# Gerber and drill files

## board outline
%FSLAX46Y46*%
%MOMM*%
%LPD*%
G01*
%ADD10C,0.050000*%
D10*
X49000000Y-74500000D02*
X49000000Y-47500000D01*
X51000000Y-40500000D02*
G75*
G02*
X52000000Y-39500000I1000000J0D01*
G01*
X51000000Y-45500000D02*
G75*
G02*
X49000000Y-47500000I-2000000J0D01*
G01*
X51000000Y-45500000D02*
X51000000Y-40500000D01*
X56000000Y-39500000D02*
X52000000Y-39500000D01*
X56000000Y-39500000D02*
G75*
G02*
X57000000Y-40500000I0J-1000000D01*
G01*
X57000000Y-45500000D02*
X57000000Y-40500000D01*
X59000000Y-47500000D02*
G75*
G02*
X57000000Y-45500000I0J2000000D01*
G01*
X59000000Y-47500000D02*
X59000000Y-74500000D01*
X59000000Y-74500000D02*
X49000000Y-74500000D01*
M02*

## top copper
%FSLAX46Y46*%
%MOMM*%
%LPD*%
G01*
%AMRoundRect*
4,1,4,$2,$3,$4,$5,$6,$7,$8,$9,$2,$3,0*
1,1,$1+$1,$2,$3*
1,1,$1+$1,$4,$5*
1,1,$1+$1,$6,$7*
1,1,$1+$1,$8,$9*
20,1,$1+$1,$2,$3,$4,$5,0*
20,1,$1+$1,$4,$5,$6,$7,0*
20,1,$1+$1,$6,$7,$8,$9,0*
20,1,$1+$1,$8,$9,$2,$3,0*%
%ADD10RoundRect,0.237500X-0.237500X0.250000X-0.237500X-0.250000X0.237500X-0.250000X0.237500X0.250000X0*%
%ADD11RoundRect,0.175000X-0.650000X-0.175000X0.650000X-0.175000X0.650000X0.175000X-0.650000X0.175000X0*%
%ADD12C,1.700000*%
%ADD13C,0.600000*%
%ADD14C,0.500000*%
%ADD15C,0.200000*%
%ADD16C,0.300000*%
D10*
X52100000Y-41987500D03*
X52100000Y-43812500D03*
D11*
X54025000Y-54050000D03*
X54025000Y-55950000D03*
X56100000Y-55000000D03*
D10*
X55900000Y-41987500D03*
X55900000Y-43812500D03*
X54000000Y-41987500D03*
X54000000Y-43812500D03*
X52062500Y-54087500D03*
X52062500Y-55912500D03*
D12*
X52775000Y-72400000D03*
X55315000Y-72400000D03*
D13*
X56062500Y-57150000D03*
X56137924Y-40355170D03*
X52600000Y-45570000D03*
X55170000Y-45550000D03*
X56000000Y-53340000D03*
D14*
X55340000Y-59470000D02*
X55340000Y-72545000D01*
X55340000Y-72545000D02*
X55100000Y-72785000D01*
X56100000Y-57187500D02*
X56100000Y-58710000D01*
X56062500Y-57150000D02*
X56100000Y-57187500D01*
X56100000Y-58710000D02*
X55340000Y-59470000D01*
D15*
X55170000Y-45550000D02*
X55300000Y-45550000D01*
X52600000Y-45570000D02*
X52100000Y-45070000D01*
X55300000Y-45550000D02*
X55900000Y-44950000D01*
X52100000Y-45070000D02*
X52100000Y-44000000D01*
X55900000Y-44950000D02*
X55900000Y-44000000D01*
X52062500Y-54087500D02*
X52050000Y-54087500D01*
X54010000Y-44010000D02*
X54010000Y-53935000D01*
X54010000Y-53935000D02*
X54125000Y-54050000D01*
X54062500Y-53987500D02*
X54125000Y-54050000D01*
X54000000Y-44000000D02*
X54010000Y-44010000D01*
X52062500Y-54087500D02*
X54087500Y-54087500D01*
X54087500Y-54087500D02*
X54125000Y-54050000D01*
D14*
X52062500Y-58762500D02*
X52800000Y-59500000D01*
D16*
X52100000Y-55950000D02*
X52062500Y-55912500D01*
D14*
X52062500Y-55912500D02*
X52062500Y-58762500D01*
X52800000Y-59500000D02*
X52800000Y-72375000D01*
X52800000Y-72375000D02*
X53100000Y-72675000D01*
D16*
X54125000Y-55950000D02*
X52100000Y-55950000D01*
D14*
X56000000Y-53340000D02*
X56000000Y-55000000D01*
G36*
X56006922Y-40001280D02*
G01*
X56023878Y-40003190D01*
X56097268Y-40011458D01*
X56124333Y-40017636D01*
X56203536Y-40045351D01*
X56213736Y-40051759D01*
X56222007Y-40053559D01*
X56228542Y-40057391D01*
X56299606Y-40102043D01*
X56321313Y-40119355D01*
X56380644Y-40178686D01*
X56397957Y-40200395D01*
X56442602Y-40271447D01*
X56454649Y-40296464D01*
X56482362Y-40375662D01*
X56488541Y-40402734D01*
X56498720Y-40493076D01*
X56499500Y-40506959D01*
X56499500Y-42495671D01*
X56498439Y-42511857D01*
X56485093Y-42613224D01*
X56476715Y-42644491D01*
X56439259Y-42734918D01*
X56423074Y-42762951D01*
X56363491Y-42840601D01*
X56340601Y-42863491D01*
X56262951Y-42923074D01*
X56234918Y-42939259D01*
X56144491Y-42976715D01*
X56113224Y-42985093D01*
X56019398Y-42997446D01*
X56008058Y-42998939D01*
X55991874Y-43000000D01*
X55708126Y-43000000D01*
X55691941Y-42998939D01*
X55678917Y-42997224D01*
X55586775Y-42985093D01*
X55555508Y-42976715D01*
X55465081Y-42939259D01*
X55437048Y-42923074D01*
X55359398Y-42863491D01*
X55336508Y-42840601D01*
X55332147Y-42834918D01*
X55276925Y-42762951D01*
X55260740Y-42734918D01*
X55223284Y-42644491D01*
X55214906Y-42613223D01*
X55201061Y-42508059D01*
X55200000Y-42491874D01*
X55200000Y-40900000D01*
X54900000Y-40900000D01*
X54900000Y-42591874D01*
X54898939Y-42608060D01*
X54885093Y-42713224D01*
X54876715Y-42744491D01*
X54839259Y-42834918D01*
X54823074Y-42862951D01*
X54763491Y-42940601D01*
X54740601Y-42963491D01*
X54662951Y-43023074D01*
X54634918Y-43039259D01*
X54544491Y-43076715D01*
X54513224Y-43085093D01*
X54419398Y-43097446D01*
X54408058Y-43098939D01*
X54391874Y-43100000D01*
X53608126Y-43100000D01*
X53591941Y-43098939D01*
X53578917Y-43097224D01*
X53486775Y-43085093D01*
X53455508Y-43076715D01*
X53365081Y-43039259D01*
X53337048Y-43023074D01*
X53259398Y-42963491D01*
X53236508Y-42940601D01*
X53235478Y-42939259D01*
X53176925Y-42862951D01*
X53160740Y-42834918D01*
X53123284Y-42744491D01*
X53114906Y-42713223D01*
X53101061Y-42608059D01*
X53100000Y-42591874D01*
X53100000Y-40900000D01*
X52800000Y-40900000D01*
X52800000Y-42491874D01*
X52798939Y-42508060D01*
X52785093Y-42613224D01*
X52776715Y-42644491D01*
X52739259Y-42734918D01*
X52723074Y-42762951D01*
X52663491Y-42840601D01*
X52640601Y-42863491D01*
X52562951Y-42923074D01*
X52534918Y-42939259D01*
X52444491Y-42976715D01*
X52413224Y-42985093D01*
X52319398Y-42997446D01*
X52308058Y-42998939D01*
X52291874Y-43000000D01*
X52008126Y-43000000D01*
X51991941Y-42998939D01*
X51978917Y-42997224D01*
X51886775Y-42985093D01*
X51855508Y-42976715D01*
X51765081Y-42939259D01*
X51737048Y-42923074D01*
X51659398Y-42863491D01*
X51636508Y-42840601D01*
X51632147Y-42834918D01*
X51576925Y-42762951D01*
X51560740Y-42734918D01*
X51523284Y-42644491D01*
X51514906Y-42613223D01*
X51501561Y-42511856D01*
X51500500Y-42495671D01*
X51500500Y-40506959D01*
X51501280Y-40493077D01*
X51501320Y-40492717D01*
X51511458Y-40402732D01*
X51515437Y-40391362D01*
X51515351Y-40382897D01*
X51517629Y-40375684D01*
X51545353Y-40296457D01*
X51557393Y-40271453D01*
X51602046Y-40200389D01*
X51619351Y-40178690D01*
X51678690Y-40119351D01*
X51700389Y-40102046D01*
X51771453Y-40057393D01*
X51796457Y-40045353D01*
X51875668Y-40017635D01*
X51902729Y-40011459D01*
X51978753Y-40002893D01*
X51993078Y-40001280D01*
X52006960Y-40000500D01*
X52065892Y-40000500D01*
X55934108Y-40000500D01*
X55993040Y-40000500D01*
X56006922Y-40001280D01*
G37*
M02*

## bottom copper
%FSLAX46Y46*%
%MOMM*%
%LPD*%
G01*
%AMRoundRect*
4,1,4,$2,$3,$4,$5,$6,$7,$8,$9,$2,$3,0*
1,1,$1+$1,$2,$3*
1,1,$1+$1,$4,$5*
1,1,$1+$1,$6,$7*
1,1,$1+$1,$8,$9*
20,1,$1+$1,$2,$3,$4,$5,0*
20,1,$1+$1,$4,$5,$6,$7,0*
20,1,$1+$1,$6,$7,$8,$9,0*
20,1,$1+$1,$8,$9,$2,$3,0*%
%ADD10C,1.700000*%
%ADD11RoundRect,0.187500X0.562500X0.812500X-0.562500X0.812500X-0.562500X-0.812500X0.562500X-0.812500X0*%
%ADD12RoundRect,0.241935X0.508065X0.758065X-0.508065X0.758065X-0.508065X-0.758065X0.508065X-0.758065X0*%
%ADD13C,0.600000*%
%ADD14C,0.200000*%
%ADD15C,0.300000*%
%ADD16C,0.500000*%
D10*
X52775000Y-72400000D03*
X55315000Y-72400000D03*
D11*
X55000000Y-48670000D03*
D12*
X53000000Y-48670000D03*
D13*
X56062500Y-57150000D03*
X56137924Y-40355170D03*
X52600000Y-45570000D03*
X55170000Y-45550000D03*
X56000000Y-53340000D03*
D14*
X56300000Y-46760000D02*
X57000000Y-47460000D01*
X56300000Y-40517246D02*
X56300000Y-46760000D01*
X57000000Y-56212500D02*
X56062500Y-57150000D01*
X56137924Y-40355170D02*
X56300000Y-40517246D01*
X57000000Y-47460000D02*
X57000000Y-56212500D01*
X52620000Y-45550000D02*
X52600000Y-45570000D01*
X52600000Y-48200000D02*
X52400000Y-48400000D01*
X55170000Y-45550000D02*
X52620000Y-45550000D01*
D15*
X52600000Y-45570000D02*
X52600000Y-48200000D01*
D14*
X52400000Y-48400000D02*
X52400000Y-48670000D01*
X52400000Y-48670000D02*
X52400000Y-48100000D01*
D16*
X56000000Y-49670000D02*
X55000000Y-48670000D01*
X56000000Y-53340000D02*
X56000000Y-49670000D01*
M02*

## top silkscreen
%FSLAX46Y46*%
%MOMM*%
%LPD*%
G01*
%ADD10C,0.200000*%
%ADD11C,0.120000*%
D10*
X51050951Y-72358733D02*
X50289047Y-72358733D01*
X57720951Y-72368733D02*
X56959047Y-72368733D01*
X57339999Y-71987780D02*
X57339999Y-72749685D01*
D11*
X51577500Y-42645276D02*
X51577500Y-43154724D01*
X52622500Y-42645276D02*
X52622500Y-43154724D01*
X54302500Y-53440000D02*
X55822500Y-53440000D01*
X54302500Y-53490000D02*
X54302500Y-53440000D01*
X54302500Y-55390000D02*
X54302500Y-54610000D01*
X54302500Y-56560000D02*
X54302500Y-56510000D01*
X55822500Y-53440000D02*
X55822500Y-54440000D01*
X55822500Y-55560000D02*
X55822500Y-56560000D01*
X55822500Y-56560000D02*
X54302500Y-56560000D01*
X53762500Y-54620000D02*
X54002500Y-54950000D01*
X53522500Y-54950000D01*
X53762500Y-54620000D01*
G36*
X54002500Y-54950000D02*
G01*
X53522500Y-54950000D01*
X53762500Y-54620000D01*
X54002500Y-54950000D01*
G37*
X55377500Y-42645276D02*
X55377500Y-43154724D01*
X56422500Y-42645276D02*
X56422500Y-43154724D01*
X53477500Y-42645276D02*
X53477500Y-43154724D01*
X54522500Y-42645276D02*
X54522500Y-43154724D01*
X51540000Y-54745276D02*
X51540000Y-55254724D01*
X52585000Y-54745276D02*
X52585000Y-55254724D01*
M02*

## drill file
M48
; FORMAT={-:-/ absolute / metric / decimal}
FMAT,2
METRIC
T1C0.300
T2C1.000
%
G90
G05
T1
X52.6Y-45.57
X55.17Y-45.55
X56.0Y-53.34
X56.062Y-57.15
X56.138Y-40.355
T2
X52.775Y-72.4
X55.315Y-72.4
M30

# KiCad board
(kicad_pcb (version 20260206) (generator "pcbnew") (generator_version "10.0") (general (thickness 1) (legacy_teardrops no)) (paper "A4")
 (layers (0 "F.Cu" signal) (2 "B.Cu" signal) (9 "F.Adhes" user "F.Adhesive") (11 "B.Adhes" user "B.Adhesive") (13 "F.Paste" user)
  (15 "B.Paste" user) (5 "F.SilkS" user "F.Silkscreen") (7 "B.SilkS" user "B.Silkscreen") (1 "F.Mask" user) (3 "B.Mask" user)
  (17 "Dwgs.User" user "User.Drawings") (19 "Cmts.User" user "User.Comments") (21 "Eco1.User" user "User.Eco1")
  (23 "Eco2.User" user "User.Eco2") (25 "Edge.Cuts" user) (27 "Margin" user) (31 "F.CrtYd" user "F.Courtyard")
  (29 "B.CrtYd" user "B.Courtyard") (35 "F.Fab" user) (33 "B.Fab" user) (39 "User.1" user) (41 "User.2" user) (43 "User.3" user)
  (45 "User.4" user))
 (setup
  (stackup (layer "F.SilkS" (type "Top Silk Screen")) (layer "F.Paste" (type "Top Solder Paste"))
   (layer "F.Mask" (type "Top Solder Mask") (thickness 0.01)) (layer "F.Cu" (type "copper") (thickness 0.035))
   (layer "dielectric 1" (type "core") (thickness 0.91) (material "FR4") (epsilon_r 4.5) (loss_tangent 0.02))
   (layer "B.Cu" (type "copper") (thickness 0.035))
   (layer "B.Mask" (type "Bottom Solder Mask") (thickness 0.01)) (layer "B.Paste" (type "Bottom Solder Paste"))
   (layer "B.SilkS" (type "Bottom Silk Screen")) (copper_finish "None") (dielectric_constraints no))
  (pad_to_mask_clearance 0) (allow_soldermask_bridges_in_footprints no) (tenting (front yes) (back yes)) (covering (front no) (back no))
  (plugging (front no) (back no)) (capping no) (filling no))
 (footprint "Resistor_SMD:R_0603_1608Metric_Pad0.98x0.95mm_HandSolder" (layer "F.Cu") (at 52.1 42.9 -90)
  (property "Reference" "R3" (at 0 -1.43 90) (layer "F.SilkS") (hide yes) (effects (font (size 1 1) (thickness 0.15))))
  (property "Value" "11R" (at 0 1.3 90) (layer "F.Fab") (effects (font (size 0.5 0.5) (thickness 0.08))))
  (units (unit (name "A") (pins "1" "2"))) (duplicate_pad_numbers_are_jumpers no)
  (fp_line (start -0.254724 0.5225) (end 0.254724 0.5225) (stroke (width 0.12) (type solid)) (layer "F.SilkS"))
  (fp_line (start -0.254724 -0.5225) (end 0.254724 -0.5225) (stroke (width 0.12) (type solid)) (layer "F.SilkS"))
  (pad "1" smd roundrect (at -0.9125 0 270) (size 0.975 0.95) (layers "F.Cu" "F.Mask" "F.Paste") (roundrect_rratio 0.25) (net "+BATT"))
  (pad "2" smd roundrect (at 0.9125 0 270) (size 0.975 0.95) (layers "F.Cu" "F.Mask" "F.Paste") (roundrect_rratio 0.25) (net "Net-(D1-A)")))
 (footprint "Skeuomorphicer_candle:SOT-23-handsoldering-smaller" (layer "F.Cu") (at 55.0625 55)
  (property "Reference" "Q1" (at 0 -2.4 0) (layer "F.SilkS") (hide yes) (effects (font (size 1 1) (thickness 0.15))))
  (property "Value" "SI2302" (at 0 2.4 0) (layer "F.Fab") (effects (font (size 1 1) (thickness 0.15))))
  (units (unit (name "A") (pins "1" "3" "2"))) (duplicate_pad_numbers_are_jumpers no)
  (fp_line (start -0.76 -1.56) (end 0.76 -1.56) (stroke (width 0.12) (type solid)) (layer "F.SilkS"))
  (fp_line (start -0.76 -1.51) (end -0.76 -1.56) (stroke (width 0.12) (type solid)) (layer "F.SilkS"))
  (fp_line (start -0.76 0.39) (end -0.76 -0.39) (stroke (width 0.12) (type solid)) (layer "F.SilkS"))
  (fp_line (start -0.76 1.56) (end -0.76 1.51) (stroke (width 0.12) (type solid)) (layer "F.SilkS"))
  (fp_line (start 0.76 -1.56) (end 0.76 -0.56) (stroke (width 0.12) (type solid)) (layer "F.SilkS"))
  (fp_line (start 0.76 0.56) (end 0.76 1.56) (stroke (width 0.12) (type solid)) (layer "F.SilkS"))
  (fp_line (start 0.76 1.56) (end -0.76 1.56) (stroke (width 0.12) (type solid)) (layer "F.SilkS"))
  (fp_poly (pts (xy -1.3 -0.38) (xy -1.06 -0.05) (xy -1.54 -0.05)) (stroke (width 0.12) (type solid)) (fill yes) (layer "F.SilkS"))
  (pad "1" smd roundrect (at -1.0375 -0.95) (size 1.65 0.7) (layers "F.Cu" "F.Mask" "F.Paste") (roundrect_rratio 0.25) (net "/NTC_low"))
  (pad "2" smd roundrect (at -1.0375 0.95) (size 1.65 0.7) (layers "F.Cu" "F.Mask" "F.Paste") (roundrect_rratio 0.25) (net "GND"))
  (pad "3" smd roundrect (at 1.0375 0) (size 1.65 0.7) (layers "F.Cu" "F.Mask" "F.Paste") (roundrect_rratio 0.25) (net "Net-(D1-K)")))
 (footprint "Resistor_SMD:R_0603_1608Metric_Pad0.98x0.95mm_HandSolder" (layer "F.Cu") (at 55.9 42.9 -90)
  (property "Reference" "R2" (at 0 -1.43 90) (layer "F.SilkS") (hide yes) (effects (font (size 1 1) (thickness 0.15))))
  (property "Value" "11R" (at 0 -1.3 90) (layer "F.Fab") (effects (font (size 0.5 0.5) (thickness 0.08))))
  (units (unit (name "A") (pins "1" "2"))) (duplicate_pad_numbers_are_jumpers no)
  (fp_line (start -0.254724 0.5225) (end 0.254724 0.5225) (stroke (width 0.12) (type solid)) (layer "F.SilkS"))
  (fp_line (start -0.254724 -0.5225) (end 0.254724 -0.5225) (stroke (width 0.12) (type solid)) (layer "F.SilkS"))
  (pad "1" smd roundrect (at -0.9125 0 270) (size 0.975 0.95) (layers "F.Cu" "F.Mask" "F.Paste") (roundrect_rratio 0.25) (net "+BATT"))
  (pad "2" smd roundrect (at 0.9125 0 270) (size 0.975 0.95) (layers "F.Cu" "F.Mask" "F.Paste") (roundrect_rratio 0.25) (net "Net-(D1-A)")))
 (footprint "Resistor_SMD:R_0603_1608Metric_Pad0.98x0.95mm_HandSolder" (layer "F.Cu") (at 54 42.9 -90)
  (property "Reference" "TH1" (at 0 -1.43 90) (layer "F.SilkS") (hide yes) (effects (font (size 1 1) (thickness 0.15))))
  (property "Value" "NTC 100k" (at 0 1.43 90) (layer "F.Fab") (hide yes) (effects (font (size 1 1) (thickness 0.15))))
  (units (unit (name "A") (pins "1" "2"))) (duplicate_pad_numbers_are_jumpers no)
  (fp_line (start -0.254724 0.5225) (end 0.254724 0.5225) (stroke (width 0.12) (type solid)) (layer "F.SilkS"))
  (fp_line (start -0.254724 -0.5225) (end 0.254724 -0.5225) (stroke (width 0.12) (type solid)) (layer "F.SilkS"))
  (pad "1" smd roundrect (at -0.9125 0 270) (size 0.975 0.95) (layers "F.Cu" "F.Mask" "F.Paste") (roundrect_rratio 0.25) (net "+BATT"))
  (pad "2" smd roundrect (at 0.9125 0 270) (size 0.975 0.95) (layers "F.Cu" "F.Mask" "F.Paste") (roundrect_rratio 0.25) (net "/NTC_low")))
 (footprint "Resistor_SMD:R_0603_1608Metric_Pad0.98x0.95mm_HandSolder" (layer "F.Cu") (at 52.0625 55 -90)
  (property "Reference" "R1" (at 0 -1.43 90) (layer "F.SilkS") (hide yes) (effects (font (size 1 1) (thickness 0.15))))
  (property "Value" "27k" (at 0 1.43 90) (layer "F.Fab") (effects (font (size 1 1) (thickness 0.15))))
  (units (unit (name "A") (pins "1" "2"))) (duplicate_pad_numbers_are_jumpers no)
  (fp_line (start -0.254724 0.5225) (end 0.254724 0.5225) (stroke (width 0.12) (type solid)) (layer "F.SilkS"))
  (fp_line (start -0.254724 -0.5225) (end 0.254724 -0.5225) (stroke (width 0.12) (type solid)) (layer "F.SilkS"))
  (pad "1" smd roundrect (at -0.9125 0 270) (size 0.975 0.95) (layers "F.Cu" "F.Mask" "F.Paste") (roundrect_rratio 0.25) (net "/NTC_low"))
  (pad "2" smd roundrect (at 0.9125 0 270) (size 0.975 0.95) (layers "F.Cu" "F.Mask" "F.Paste") (roundrect_rratio 0.25) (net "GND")))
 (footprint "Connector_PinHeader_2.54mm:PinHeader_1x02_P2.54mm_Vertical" (layer "F.Cu") (at 52.775 72.4 90)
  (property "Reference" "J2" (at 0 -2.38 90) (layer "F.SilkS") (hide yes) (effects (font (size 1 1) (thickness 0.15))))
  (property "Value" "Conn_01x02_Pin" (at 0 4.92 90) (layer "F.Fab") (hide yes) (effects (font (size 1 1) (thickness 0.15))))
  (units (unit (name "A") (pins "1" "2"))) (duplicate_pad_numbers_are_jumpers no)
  (pad "1" thru_hole circle (at 0 0 90) (size 1.7 1.7) (drill 1) (layers "*.Cu" "*.Mask") (remove_unused_layers no) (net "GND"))
  (pad "2" thru_hole circle (at 0 2.54 90) (size 1.7 1.7) (drill 1) (layers "*.Cu" "*.Mask") (remove_unused_layers no) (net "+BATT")))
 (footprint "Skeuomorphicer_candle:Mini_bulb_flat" (layer "B.Cu") (at 54 48.67 180)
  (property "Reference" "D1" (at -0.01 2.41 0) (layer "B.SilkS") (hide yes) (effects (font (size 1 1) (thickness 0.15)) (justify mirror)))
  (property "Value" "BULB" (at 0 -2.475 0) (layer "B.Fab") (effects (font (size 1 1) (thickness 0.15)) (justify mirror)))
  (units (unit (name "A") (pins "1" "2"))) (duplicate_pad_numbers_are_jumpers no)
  (pad "1" smd roundrect (at -1 0 180) (size 1.5 2) (layers "B.Cu" "B.Mask" "B.Paste") (roundrect_rratio 0.125) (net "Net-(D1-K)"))
  (pad "2" smd roundrect (at 1 0 180) (size 1.5 2) (layers "B.Cu" "B.Mask" "B.Paste") (roundrect_rratio 0.1612903226) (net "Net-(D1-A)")))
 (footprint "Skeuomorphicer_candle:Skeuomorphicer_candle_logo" (layer "B.Cu") (at 53.94 63.23 180)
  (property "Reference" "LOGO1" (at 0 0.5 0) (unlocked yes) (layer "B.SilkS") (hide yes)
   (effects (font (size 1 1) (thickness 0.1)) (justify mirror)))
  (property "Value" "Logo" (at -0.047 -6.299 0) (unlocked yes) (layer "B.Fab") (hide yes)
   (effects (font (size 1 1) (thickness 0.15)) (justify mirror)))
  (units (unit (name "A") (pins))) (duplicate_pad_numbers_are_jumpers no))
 (gr_line (start 49 74.5) (end 49 47.5) (stroke (width 0.05) (type default)) (layer "Edge.Cuts"))
 (gr_arc (start 51 40.5) (mid 51.292893 39.792893) (end 52 39.5) (stroke (width 0.05) (type default)) (layer "Edge.Cuts"))
 (gr_arc (start 51 45.5) (mid 50.414214 46.914214) (end 49 47.5) (stroke (width 0.05) (type default)) (layer "Edge.Cuts"))
 (gr_line (start 51 45.5) (end 51 40.5) (stroke (width 0.05) (type default)) (layer "Edge.Cuts"))
 (gr_line (start 56 39.5) (end 52 39.5) (stroke (width 0.05) (type default)) (layer "Edge.Cuts"))
 (gr_arc (start 56 39.5) (mid 56.707107 39.792893) (end 57 40.5) (stroke (width 0.05) (type default)) (layer "Edge.Cuts"))
 (gr_line (start 57 45.5) (end 57 40.5) (stroke (width 0.05) (type default)) (layer "Edge.Cuts"))
 (gr_arc (start 59 47.5) (mid 57.585786 46.914214) (end 57 45.5) (stroke (width 0.05) (type default)) (layer "Edge.Cuts"))
 (gr_line (start 59 47.5) (end 59 74.5) (stroke (width 0.05) (type default)) (layer "Edge.Cuts"))
 (gr_line (start 59 74.5) (end 49 74.5) (stroke (width 0.05) (type default)) (layer "Edge.Cuts"))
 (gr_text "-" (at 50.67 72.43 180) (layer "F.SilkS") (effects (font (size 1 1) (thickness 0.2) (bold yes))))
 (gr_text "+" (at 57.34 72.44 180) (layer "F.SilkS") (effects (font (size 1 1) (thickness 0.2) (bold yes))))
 (segment (start 55.34 59.47) (end 55.34 72.545) (width 0.5) (layer "F.Cu") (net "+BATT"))
 (segment (start 55.34 72.545) (end 55.1 72.785) (width 0.5) (layer "F.Cu") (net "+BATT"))
 (segment (start 56.1 57.1875) (end 56.1 58.71) (width 0.5) (layer "F.Cu") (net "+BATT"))
 (segment (start 56.0625 57.15) (end 56.1 57.1875) (width 0.5) (layer "F.Cu") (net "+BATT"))
 (segment (start 56.1 58.71) (end 55.34 59.47) (width 0.5) (layer "F.Cu") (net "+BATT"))
 (via (at 56.0625 57.15) (size 0.6) (drill 0.3) (layers "F.Cu" "B.Cu") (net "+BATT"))
 (via (at 56.137924 40.35517) (size 0.6) (drill 0.3) (layers "F.Cu" "B.Cu") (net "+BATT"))
 (segment (start 56.3 46.76) (end 57 47.46) (width 0.2) (layer "B.Cu") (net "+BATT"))
 (segment (start 56.3 40.517246) (end 56.3 46.76) (width 0.2) (layer "B.Cu") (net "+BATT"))
 (segment (start 57 56.2125) (end 56.0625 57.15) (width 0.2) (layer "B.Cu") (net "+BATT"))
 (segment (start 56.137924 40.35517) (end 56.3 40.517246) (width 0.2) (layer "B.Cu") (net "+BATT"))
 (segment (start 57 47.46) (end 57 56.2125) (width 0.2) (layer "B.Cu") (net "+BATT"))
 (segment (start 55.17 45.55) (end 55.3 45.55) (width 0.2) (layer "F.Cu") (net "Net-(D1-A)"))
 (segment (start 52.6 45.57) (end 52.1 45.07) (width 0.2) (layer "F.Cu") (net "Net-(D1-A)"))
 (segment (start 55.3 45.55) (end 55.9 44.95) (width 0.2) (layer "F.Cu") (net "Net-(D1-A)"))
 (segment (start 52.1 45.07) (end 52.1 44) (width 0.2) (layer "F.Cu") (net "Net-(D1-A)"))
 (segment (start 55.9 44.95) (end 55.9 44) (width 0.2) (layer "F.Cu") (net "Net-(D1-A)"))
 (via (at 52.6 45.57) (size 0.6) (drill 0.3) (layers "F.Cu" "B.Cu") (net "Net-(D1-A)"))
 (via (at 55.17 45.55) (size 0.6) (drill 0.3) (layers "F.Cu" "B.Cu") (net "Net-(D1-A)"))
 (segment (start 52.62 45.55) (end 52.6 45.57) (width 0.2) (layer "B.Cu") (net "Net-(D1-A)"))
 (segment (start 52.6 48.2) (end 52.4 48.4) (width 0.2) (layer "B.Cu") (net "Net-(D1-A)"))
 (segment (start 55.17 45.55) (end 52.62 45.55) (width 0.2) (layer "B.Cu") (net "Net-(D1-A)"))
 (segment (start 52.6 45.57) (end 52.6 48.2) (width 0.3) (layer "B.Cu") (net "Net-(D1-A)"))
 (segment (start 52.4 48.4) (end 52.4 48.67) (width 0.2) (layer "B.Cu") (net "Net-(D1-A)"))
 (segment (start 52.4 48.67) (end 52.4 48.1) (width 0.2) (layer "B.Cu") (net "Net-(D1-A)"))
 (segment (start 52.0625 54.0875) (end 52.05 54.0875) (width 0.2) (layer "F.Cu") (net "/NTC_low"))
 (segment (start 54.01 44.01) (end 54.01 53.935) (width 0.2) (layer "F.Cu") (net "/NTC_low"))
 (segment (start 54.01 53.935) (end 54.125 54.05) (width 0.2) (layer "F.Cu") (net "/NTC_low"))
 (segment (start 54.0625 53.9875) (end 54.125 54.05) (width 0.2) (layer "F.Cu") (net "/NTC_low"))
 (segment (start 54 44) (end 54.01 44.01) (width 0.2) (layer "F.Cu") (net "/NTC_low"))
 (segment (start 52.0625 54.0875) (end 54.0875 54.0875) (width 0.2) (layer "F.Cu") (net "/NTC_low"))
 (segment (start 54.0875 54.0875) (end 54.125 54.05) (width 0.2) (layer "F.Cu") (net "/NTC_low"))
 (segment (start 52.0625 58.7625) (end 52.8 59.5) (width 0.5) (layer "F.Cu") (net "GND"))
 (segment (start 52.1 55.95) (end 52.0625 55.9125) (width 0.3) (layer "F.Cu") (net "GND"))
 (segment (start 52.0625 55.9125) (end 52.0625 58.7625) (width 0.5) (layer "F.Cu") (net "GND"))
 (segment (start 52.8 59.5) (end 52.8 72.375) (width 0.5) (layer "F.Cu") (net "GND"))
 (segment (start 52.8 72.375) (end 53.1 72.675) (width 0.5) (layer "F.Cu") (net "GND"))
 (segment (start 54.125 55.95) (end 52.1 55.95) (width 0.3) (layer "F.Cu") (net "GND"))
 (segment (start 56 53.34) (end 56 55) (width 0.5) (layer "F.Cu") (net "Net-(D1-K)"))
 (via (at 56 53.34) (size 0.6) (drill 0.3) (layers "F.Cu" "B.Cu") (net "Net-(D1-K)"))
 (segment (start 56 49.67) (end 55 48.67) (width 0.5) (layer "B.Cu") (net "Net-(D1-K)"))
 (segment (start 56 53.34) (end 56 49.67) (width 0.5) (layer "B.Cu") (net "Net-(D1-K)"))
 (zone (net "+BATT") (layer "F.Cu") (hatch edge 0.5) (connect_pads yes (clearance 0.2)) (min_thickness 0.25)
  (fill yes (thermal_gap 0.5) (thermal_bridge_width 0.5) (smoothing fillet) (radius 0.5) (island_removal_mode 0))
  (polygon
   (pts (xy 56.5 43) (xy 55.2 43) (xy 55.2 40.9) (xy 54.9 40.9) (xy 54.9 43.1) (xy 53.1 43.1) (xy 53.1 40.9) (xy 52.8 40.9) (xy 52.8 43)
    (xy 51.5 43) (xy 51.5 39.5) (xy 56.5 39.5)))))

